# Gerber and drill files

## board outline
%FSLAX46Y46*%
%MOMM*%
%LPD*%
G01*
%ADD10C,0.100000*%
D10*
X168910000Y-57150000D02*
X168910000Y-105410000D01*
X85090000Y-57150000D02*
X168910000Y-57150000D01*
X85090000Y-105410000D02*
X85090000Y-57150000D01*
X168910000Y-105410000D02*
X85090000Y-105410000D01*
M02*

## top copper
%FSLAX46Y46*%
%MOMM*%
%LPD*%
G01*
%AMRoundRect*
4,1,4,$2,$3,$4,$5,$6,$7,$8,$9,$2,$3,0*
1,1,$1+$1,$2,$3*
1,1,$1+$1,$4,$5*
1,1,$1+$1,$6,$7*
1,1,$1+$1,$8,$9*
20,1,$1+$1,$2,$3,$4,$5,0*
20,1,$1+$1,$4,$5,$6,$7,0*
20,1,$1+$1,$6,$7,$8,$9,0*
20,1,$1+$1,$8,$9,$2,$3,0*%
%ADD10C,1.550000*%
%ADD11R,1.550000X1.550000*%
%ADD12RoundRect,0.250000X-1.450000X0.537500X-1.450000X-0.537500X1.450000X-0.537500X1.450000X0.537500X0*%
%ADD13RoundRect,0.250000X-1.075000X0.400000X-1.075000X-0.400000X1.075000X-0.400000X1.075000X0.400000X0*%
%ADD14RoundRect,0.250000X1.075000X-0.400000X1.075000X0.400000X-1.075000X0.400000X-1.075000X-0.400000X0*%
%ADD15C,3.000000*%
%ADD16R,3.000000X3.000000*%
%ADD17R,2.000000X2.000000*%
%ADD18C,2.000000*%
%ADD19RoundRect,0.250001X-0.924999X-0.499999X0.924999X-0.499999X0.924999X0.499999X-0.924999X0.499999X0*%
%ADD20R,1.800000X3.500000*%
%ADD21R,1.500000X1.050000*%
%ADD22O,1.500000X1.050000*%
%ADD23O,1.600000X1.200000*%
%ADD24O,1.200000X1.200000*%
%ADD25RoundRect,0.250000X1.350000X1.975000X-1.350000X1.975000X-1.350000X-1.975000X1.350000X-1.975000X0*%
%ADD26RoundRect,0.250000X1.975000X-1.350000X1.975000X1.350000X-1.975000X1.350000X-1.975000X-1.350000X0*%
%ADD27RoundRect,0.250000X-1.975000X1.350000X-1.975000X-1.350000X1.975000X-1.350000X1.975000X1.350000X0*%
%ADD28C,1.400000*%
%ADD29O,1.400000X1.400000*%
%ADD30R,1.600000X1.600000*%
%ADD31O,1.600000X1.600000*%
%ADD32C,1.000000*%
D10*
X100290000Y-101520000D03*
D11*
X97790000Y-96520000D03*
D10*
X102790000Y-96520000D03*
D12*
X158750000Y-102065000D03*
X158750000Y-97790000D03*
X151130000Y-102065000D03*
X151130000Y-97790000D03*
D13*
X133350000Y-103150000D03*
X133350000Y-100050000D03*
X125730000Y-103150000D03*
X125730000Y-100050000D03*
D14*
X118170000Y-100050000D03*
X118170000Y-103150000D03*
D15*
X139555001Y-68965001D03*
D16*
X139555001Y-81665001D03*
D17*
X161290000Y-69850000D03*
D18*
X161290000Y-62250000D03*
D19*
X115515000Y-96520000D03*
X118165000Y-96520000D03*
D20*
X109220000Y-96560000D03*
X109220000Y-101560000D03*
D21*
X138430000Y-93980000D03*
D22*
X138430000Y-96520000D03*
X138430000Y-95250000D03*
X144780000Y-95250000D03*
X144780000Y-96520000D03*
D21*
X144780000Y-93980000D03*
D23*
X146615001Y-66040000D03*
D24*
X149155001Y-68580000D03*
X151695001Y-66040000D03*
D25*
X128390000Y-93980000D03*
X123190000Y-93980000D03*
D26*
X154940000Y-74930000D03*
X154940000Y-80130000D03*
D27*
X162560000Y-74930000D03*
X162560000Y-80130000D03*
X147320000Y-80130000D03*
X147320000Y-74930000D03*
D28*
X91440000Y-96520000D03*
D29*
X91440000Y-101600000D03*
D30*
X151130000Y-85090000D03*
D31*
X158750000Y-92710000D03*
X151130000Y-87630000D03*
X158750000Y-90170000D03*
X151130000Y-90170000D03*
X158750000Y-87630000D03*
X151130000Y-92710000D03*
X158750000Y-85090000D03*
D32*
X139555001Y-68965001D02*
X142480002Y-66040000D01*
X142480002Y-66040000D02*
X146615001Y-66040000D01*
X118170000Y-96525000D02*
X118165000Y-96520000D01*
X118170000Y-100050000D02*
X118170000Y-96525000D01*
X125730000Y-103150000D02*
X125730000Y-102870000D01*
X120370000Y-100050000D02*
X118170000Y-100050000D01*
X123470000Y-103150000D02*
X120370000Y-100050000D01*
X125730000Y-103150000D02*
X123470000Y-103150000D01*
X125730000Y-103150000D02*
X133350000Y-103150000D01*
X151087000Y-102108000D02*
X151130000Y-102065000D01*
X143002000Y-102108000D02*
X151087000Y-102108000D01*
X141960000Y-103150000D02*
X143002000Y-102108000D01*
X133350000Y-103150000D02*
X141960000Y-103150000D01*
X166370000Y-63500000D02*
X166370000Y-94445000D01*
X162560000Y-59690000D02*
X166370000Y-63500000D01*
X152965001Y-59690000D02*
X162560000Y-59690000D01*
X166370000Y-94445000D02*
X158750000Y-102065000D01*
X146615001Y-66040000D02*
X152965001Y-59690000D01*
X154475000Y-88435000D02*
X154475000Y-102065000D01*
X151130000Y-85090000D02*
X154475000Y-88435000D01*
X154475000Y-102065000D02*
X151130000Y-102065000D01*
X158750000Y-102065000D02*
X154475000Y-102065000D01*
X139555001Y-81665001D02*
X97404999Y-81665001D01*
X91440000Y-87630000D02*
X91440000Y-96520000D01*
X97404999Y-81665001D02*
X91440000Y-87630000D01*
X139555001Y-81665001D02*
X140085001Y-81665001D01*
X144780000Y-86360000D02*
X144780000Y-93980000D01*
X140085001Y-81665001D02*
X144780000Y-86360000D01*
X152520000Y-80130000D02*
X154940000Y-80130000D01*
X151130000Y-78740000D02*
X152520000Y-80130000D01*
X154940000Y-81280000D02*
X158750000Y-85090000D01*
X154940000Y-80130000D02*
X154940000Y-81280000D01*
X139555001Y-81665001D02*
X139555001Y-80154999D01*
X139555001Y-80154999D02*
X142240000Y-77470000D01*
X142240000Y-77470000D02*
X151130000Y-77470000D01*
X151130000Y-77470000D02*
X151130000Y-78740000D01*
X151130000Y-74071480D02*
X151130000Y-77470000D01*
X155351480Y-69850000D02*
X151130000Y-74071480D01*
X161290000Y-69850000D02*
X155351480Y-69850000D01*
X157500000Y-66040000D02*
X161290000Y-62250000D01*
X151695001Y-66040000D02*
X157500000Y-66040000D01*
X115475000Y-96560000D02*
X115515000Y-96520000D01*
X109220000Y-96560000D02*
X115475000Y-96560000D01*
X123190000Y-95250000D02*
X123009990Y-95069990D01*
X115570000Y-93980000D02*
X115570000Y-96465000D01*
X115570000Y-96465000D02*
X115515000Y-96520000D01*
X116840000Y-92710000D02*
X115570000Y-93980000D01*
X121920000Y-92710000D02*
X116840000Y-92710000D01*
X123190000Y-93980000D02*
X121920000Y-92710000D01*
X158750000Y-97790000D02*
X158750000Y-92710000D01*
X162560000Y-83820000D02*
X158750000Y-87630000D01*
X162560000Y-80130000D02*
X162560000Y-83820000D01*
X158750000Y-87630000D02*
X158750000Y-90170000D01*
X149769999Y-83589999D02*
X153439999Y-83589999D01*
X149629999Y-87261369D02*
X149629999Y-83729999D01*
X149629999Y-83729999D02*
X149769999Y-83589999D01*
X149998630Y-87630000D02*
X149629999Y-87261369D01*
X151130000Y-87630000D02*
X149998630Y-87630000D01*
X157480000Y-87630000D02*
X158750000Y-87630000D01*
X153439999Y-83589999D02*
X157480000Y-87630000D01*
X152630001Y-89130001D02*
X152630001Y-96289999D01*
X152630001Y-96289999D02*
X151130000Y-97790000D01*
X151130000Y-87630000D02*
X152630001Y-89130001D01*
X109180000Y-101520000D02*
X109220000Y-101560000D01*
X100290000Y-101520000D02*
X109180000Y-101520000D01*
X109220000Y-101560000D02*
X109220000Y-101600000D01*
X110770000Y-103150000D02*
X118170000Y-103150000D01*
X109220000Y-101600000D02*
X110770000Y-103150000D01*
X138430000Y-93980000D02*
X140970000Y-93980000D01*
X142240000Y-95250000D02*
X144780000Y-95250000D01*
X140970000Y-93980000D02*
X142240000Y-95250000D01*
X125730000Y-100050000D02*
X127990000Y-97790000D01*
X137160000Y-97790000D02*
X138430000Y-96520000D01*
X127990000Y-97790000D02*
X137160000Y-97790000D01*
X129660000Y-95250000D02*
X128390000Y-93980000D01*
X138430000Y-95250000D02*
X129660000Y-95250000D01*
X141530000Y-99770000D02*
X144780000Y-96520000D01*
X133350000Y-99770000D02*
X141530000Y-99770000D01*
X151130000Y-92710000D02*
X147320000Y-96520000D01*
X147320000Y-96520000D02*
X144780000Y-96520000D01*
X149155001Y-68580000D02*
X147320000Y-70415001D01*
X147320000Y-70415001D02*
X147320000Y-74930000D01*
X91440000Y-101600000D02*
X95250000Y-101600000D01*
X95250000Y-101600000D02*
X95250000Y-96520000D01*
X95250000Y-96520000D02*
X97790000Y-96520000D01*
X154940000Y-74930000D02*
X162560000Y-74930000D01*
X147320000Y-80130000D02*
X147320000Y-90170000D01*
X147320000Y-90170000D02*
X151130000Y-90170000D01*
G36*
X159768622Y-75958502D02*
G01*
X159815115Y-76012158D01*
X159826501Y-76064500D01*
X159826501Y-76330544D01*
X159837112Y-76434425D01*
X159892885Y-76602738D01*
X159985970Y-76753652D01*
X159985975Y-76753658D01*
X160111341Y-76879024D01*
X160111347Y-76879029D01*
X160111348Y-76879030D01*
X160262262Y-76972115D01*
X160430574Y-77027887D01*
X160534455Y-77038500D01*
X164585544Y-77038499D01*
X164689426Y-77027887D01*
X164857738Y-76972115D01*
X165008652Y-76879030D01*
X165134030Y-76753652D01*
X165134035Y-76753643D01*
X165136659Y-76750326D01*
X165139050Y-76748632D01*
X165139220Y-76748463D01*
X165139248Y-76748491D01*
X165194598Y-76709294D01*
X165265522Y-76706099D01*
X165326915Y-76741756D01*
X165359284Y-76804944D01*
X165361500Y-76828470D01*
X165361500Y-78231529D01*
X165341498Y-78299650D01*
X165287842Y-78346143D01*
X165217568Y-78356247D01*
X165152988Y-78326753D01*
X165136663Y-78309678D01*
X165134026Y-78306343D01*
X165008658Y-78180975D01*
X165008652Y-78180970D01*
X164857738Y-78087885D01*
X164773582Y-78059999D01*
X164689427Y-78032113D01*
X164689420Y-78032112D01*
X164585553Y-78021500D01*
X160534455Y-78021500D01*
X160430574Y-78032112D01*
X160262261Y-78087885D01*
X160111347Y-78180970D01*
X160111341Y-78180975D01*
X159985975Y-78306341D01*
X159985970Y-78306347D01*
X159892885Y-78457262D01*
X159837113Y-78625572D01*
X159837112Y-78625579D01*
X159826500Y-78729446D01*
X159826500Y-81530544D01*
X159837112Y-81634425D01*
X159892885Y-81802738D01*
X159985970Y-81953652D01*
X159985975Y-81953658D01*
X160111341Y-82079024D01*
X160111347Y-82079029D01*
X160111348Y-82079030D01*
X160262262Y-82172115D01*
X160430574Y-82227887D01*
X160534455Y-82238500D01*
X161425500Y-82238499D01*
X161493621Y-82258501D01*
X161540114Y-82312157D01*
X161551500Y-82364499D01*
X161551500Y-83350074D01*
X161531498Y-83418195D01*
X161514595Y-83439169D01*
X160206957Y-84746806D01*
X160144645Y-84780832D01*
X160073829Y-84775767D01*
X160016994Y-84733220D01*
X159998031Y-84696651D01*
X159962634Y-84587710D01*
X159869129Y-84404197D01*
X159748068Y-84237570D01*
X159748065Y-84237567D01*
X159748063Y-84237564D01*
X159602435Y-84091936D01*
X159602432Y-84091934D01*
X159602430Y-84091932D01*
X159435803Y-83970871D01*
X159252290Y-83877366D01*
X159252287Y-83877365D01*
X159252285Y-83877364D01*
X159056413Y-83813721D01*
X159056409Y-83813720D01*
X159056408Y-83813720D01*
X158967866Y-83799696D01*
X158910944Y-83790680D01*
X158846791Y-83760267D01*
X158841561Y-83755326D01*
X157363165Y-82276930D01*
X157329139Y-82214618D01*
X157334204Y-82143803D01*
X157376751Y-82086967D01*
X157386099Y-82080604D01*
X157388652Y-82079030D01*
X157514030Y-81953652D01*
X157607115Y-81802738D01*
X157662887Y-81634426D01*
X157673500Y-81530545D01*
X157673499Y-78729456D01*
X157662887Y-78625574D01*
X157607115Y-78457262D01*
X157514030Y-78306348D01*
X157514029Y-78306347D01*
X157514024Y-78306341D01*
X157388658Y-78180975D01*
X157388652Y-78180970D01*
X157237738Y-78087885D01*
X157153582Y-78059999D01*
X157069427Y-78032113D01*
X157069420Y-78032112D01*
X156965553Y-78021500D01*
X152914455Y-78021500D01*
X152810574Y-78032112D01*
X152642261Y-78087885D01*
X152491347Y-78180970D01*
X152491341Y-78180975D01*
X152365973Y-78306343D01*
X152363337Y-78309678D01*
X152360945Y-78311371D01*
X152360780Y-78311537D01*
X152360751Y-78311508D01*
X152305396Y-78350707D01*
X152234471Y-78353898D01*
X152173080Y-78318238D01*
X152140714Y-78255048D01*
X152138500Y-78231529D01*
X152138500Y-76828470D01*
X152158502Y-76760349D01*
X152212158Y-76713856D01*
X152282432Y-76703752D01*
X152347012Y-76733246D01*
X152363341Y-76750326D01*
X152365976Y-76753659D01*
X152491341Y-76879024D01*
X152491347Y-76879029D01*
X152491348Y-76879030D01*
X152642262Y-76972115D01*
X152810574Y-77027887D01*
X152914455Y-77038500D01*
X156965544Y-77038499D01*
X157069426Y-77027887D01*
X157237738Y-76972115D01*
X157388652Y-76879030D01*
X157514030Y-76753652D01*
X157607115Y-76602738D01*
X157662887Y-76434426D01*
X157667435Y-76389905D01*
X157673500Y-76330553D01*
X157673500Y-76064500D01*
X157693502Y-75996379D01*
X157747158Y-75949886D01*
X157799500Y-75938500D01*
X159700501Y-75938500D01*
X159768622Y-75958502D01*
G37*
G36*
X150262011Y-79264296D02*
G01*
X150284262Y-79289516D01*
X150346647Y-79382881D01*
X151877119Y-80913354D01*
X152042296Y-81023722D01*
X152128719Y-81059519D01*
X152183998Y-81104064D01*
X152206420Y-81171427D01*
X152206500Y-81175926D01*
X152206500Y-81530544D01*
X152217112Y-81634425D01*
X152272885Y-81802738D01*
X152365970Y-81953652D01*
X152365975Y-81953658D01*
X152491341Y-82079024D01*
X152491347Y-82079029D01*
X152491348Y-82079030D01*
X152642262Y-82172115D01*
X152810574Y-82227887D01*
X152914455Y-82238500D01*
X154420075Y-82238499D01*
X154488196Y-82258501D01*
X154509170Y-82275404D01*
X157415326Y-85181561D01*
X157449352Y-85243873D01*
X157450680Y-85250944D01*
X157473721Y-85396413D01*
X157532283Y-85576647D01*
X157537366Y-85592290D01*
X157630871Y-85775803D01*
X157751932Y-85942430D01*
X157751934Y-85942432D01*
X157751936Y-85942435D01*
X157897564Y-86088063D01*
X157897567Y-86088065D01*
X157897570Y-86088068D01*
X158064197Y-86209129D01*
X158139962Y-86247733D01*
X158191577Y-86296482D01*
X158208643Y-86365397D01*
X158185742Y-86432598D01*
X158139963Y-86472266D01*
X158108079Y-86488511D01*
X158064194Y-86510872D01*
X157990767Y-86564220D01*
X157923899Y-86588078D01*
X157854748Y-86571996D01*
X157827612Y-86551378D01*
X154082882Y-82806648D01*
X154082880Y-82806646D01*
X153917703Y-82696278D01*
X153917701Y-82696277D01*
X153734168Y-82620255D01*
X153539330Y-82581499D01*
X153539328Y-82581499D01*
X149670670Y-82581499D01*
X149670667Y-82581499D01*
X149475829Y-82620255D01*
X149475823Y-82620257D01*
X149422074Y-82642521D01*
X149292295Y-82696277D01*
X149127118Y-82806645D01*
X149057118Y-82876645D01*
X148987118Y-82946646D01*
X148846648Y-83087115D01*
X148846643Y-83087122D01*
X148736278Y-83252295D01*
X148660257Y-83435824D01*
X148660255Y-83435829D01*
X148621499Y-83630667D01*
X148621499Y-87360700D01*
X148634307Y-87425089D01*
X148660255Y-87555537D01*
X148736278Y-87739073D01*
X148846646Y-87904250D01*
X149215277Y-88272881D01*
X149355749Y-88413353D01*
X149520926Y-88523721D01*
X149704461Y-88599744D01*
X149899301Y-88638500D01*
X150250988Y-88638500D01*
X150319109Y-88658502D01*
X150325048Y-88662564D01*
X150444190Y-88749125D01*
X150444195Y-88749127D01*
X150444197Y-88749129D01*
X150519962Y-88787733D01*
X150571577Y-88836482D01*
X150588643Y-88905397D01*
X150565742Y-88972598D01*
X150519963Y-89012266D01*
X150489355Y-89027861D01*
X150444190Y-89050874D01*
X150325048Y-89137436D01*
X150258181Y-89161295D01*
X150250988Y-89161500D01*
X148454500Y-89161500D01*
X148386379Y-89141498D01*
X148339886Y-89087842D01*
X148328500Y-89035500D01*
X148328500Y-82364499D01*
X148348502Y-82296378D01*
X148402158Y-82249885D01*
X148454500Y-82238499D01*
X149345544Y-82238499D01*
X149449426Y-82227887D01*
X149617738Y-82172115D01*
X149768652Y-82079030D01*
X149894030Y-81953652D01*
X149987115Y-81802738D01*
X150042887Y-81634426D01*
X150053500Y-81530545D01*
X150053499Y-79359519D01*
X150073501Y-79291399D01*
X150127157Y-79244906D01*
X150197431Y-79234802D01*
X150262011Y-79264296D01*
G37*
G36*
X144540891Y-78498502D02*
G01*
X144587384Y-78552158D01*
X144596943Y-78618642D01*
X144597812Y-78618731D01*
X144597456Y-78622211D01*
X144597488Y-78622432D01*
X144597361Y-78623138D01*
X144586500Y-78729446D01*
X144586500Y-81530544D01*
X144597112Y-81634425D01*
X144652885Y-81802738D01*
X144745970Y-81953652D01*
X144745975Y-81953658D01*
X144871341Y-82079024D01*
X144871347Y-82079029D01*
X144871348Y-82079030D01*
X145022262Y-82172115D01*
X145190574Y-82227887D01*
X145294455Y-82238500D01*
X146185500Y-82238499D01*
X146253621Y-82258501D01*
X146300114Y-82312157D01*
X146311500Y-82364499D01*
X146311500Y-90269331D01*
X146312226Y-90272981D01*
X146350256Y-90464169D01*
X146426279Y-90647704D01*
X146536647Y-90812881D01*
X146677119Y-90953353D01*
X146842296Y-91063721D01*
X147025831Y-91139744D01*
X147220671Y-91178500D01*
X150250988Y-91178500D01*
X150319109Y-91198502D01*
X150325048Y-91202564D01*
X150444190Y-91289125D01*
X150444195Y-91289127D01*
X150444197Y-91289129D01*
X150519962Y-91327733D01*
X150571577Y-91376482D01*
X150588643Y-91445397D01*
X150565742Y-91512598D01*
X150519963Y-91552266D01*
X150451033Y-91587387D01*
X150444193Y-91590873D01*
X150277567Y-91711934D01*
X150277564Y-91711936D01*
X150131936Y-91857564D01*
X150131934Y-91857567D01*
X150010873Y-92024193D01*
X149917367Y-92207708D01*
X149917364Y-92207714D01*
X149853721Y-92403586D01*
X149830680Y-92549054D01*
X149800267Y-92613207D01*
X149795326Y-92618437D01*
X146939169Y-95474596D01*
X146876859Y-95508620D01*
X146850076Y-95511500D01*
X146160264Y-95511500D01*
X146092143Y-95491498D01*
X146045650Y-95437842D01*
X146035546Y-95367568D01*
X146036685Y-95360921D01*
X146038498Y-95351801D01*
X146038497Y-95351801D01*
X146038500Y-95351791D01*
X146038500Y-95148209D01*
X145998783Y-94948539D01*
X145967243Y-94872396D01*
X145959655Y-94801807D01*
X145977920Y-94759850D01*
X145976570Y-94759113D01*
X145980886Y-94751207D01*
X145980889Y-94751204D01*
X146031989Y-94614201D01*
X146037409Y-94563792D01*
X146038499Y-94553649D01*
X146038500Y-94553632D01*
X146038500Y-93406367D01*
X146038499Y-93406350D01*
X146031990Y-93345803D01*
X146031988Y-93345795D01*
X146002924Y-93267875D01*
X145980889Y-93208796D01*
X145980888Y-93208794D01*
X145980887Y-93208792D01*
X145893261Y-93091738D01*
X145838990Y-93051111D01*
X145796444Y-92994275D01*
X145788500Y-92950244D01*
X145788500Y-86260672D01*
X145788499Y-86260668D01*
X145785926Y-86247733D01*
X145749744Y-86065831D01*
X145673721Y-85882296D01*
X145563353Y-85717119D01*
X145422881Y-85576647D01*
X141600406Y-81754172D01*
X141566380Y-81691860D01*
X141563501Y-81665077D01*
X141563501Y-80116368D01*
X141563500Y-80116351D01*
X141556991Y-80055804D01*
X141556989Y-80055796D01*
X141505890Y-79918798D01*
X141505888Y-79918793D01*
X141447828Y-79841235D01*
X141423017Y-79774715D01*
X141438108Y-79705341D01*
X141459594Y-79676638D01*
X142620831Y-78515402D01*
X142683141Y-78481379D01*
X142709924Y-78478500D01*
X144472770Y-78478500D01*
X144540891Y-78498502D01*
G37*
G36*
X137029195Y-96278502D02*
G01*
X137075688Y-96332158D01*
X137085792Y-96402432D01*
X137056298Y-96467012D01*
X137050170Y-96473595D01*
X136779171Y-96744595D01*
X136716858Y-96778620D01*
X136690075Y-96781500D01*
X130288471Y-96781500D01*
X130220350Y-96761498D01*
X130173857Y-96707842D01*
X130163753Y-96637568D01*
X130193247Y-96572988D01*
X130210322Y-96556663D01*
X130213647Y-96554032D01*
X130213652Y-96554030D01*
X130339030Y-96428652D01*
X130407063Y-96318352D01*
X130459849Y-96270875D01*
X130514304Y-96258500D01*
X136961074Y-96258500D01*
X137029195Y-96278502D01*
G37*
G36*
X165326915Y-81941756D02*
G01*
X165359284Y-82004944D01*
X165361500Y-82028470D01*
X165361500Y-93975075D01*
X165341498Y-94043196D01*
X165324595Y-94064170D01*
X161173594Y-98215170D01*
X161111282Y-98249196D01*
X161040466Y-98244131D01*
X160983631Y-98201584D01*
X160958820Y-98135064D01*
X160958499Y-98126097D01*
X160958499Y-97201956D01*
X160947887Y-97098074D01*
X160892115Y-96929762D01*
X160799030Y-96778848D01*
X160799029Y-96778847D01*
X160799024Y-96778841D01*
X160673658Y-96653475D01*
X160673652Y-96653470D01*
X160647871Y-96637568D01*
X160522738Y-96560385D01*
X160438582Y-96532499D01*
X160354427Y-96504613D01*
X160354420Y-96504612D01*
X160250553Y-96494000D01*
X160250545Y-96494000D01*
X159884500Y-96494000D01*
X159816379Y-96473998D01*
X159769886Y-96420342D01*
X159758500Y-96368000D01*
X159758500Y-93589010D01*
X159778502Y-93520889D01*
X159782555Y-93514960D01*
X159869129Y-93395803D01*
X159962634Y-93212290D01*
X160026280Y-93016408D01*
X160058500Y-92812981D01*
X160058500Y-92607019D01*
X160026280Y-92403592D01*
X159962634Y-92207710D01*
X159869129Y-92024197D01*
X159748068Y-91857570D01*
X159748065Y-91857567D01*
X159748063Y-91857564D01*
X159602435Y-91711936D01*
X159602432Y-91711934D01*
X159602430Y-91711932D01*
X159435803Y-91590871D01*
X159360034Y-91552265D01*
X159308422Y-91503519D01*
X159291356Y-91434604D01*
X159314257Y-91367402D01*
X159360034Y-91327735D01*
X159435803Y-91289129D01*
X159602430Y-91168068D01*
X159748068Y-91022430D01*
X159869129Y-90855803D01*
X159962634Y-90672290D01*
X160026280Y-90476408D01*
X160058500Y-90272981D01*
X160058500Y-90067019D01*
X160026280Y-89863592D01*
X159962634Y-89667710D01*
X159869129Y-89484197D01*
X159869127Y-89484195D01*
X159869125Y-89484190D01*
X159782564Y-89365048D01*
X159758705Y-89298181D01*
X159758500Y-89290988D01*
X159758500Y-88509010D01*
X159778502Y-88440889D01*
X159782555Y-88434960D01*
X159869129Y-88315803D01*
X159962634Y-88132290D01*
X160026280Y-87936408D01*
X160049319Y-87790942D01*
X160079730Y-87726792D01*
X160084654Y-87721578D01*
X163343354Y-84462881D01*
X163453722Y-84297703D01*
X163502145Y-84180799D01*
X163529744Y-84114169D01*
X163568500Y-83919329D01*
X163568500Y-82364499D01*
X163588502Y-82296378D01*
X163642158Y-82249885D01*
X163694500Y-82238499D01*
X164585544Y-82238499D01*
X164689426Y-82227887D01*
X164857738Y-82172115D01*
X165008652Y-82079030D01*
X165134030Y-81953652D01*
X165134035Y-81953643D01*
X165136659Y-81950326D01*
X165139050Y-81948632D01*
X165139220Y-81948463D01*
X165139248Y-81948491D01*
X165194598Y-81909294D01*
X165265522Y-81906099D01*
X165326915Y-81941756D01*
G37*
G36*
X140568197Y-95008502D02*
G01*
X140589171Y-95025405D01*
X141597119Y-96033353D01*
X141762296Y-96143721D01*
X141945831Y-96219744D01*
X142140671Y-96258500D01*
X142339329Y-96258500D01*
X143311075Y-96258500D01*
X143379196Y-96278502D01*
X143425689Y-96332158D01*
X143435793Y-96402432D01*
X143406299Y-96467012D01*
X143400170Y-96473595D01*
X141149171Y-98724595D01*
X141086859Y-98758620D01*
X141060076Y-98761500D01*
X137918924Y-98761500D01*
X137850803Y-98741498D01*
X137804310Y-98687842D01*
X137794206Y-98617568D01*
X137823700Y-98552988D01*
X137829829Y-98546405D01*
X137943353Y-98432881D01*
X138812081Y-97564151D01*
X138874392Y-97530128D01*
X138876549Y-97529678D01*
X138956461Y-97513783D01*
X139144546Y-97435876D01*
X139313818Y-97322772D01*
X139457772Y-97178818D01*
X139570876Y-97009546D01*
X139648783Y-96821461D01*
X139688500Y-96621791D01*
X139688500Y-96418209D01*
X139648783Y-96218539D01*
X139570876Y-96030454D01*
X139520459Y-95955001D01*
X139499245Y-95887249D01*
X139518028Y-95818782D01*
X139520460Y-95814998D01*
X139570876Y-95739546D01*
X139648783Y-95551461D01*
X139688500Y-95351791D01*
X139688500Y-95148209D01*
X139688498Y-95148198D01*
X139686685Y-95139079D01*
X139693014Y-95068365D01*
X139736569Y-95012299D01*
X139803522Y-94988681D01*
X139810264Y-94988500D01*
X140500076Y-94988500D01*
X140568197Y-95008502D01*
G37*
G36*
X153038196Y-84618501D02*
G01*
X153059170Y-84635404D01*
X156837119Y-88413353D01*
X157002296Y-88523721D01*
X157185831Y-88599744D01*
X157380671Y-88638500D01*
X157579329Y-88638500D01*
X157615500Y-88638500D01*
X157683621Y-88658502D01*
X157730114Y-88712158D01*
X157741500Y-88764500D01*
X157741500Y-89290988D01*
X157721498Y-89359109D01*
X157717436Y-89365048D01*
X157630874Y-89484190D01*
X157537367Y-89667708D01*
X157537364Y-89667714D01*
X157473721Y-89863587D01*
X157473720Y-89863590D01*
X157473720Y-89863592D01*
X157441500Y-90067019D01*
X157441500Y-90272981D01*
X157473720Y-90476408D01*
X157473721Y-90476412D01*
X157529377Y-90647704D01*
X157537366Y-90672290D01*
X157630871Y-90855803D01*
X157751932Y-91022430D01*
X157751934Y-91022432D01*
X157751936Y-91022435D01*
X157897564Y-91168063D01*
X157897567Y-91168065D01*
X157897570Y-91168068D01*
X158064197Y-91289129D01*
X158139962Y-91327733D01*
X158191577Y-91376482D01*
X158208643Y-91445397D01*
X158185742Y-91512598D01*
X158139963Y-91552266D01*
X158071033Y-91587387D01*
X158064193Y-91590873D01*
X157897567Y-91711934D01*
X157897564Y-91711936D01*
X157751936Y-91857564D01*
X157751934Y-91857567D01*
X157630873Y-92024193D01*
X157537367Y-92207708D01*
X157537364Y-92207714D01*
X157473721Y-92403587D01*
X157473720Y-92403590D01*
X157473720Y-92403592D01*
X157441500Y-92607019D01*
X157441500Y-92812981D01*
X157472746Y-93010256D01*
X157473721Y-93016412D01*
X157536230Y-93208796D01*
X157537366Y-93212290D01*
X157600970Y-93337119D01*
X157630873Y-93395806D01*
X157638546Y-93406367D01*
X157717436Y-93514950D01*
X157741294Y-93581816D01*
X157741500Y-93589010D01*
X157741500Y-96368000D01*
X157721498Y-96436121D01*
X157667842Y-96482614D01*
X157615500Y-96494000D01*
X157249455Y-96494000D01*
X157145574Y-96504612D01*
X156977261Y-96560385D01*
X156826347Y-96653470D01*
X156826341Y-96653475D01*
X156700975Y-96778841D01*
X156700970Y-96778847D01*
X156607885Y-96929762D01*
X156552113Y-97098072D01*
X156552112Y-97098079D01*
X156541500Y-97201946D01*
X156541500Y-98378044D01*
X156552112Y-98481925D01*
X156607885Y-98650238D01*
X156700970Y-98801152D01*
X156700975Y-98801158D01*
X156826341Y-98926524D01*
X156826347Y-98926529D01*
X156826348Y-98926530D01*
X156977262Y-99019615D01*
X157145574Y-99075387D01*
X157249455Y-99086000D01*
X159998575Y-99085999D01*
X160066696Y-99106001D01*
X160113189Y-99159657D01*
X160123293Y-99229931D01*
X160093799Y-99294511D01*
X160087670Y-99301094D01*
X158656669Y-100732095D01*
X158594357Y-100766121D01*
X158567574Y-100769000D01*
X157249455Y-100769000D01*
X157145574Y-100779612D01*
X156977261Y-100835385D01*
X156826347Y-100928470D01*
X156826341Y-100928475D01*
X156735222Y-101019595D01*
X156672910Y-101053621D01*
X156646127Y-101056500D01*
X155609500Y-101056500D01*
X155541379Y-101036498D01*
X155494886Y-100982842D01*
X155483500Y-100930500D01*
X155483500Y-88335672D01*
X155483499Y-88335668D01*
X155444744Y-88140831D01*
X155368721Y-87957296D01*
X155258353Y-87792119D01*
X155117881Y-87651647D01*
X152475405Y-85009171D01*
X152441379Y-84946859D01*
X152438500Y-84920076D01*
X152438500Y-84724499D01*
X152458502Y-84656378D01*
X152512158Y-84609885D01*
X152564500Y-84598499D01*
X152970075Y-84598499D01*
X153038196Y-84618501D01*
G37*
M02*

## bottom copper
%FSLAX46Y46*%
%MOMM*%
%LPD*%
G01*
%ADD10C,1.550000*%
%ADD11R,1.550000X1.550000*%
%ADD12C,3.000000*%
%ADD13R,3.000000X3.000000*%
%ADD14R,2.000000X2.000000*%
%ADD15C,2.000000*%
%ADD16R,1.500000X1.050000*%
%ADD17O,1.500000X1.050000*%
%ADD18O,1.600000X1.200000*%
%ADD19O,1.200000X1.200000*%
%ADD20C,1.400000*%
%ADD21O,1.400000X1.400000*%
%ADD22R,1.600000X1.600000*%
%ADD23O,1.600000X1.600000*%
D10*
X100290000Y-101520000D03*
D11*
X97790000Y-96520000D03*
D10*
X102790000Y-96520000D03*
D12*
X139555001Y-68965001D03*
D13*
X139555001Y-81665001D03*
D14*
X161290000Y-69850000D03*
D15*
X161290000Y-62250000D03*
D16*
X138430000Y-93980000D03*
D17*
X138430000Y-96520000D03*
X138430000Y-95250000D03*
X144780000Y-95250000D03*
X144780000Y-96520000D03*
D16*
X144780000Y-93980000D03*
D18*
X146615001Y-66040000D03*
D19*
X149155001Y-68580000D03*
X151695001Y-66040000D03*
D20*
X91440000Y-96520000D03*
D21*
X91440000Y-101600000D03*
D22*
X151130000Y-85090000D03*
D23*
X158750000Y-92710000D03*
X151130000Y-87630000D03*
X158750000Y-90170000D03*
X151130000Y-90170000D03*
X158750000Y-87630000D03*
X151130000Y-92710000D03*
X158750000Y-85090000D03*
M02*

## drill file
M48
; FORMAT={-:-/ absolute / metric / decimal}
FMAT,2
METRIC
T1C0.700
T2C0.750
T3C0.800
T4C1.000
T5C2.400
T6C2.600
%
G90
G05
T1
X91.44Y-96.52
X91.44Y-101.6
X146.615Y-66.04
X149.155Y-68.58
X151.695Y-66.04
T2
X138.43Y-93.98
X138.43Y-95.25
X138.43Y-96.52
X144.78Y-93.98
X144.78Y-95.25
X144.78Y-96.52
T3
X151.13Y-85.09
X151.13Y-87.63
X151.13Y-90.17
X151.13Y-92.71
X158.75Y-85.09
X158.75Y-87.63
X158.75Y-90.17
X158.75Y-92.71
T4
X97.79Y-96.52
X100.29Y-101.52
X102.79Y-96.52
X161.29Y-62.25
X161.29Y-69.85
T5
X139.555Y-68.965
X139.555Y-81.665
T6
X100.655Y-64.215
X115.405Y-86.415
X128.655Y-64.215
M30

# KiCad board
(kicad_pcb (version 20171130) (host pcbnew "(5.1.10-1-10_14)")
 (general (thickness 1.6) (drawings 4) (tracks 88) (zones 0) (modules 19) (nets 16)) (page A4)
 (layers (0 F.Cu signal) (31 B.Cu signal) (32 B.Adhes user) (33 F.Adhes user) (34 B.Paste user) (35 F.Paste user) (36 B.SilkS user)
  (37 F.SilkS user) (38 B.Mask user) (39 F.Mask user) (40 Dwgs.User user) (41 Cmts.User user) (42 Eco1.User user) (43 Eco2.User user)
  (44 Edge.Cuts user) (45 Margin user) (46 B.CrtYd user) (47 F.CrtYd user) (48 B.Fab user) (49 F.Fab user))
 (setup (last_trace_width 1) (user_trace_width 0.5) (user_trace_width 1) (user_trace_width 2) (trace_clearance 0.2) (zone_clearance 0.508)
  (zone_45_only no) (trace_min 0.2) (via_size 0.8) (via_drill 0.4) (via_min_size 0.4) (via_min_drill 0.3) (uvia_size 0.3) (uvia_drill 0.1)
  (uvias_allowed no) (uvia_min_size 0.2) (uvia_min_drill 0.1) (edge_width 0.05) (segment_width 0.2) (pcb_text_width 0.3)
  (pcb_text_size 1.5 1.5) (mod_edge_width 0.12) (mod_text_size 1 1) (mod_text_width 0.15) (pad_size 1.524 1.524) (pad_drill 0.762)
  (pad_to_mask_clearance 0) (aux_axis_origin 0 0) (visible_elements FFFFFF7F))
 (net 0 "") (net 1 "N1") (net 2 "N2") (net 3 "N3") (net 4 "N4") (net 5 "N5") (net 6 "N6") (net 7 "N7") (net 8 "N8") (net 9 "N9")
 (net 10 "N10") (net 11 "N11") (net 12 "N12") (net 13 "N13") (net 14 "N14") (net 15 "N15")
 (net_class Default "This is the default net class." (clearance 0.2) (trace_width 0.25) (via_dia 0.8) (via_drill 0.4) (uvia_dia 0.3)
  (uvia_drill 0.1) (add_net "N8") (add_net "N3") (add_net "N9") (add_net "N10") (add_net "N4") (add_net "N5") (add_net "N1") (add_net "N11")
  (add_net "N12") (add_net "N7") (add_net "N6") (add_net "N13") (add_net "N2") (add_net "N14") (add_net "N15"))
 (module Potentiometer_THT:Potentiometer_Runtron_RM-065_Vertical (layer F.Cu) (at 97.79 96.52)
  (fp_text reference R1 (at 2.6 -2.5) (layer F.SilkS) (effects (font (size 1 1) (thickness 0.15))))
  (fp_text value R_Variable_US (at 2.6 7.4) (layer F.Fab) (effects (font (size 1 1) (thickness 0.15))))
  (pad 2 thru_hole circle (at 2.5 5) (size 1.55 1.55) (drill 1) (layers *.Cu *.Mask) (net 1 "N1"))
  (pad 1 thru_hole rect (at 0 0) (size 1.55 1.55) (drill 1) (layers *.Cu *.Mask) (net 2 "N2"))
  (pad 3 thru_hole circle (at 5 0) (size 1.55 1.55) (drill 1) (layers *.Cu *.Mask)))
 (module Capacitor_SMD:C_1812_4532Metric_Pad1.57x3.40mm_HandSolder (layer F.Cu) (at 158.75 99.9275 270)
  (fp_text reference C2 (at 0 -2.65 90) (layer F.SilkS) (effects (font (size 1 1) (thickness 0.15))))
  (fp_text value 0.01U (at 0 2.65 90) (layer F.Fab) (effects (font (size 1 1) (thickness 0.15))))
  (pad 2 smd roundrect (at 2.1375 0 270) (size 1.575 3.4) (layers F.Cu F.Paste F.Mask) (roundrect_rratio 0.15873) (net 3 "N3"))
  (pad 1 smd roundrect (at -2.1375 0 270) (size 1.575 3.4) (layers F.Cu F.Paste F.Mask) (roundrect_rratio 0.15873) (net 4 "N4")))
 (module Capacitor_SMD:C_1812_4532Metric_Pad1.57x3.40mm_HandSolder (layer F.Cu) (at 151.13 99.9275 270)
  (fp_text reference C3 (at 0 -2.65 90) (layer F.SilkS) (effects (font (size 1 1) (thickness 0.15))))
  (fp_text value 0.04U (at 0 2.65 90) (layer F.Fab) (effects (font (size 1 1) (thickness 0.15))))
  (pad 2 smd roundrect (at 2.1375 0 270) (size 1.575 3.4) (layers F.Cu F.Paste F.Mask) (roundrect_rratio 0.15873) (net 3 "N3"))
  (pad 1 smd roundrect (at -2.1375 0 270) (size 1.575 3.4) (layers F.Cu F.Paste F.Mask) (roundrect_rratio 0.15873) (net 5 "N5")))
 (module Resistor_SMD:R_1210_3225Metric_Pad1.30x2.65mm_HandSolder (layer F.Cu) (at 133.35 101.6 270)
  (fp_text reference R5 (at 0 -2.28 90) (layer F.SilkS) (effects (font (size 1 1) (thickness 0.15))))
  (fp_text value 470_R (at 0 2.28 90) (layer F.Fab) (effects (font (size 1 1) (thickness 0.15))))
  (pad 2 smd roundrect (at 1.55 0 270) (size 1.3 2.65) (layers F.Cu F.Paste F.Mask) (roundrect_rratio 0.192308) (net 3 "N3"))
  (pad 1 smd roundrect (at -1.55 0 270) (size 1.3 2.65) (layers F.Cu F.Paste F.Mask) (roundrect_rratio 0.192308) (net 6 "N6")))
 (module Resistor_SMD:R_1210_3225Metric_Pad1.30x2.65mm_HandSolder (layer F.Cu) (at 125.73 101.6 270)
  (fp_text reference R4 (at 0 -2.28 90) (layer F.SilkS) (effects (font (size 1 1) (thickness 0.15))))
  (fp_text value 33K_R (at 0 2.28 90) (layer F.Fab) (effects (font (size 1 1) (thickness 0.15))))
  (pad 2 smd roundrect (at 1.55 0 270) (size 1.3 2.65) (layers F.Cu F.Paste F.Mask) (roundrect_rratio 0.192308) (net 3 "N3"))
  (pad 1 smd roundrect (at -1.55 0 270) (size 1.3 2.65) (layers F.Cu F.Paste F.Mask) (roundrect_rratio 0.192308) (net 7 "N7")))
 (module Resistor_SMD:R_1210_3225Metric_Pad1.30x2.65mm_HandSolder (layer F.Cu) (at 118.17 101.6 90)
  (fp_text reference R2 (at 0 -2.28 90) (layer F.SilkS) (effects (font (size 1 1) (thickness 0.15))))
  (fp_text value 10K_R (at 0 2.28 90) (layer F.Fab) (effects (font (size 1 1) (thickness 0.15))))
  (pad 2 smd roundrect (at 1.55 0 90) (size 1.3 2.65) (layers F.Cu F.Paste F.Mask) (roundrect_rratio 0.192308) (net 3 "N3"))
  (pad 1 smd roundrect (at -1.55 0 90) (size 1.3 2.65) (layers F.Cu F.Paste F.Mask) (roundrect_rratio 0.192308) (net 1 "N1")))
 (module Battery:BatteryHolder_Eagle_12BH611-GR (layer F.Cu) (at 139.555001 81.665001)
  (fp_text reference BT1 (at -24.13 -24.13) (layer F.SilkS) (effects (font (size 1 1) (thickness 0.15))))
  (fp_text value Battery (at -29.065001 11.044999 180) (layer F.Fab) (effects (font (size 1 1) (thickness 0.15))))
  (pad 2 thru_hole circle (at 0 -12.7) (size 3 3) (drill 2.4) (layers *.Cu *.Mask) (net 3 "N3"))
  (pad 1 thru_hole rect (at 0 0) (size 3 3) (drill 2.4) (layers *.Cu *.Mask) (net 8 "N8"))
  (pad "" np_thru_hole circle (at -10.9 -17.45) (size 2.6 2.6) (drill 2.6) (layers *.Cu *.Mask))
  (pad "" np_thru_hole circle (at -38.9 -17.45) (size 2.6 2.6) (drill 2.6) (layers *.Cu *.Mask))
  (pad "" np_thru_hole circle (at -24.15 4.75) (size 2.6 2.6) (drill 2.6) (layers *.Cu *.Mask)))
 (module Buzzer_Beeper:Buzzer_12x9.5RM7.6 (layer F.Cu) (at 161.29 69.85 90)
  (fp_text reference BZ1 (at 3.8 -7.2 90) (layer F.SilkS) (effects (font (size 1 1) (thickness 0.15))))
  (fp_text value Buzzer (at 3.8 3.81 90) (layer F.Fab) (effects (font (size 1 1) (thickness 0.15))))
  (pad 1 thru_hole rect (at 0 0 90) (size 2 2) (drill 1) (layers *.Cu *.Mask) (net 8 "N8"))
  (pad 2 thru_hole circle (at 7.6 0 90) (size 2 2) (drill 1) (layers *.Cu *.Mask) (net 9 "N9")))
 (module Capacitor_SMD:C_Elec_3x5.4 (layer F.Cu) (at 116.84 96.52)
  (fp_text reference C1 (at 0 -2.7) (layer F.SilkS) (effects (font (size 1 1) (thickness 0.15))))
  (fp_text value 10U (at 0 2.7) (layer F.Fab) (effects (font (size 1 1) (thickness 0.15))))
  (pad 1 smd roundrect (at -1.325 0) (size 2.35 1.5) (layers F.Cu F.Paste F.Mask) (roundrect_rratio 0.166667) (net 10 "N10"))
  (pad 2 smd roundrect (at 1.325 0) (size 2.35 1.5) (layers F.Cu F.Paste F.Mask) (roundrect_rratio 0.166667) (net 3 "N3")))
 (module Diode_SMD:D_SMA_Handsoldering (layer F.Cu) (at 109.22 99.06 270)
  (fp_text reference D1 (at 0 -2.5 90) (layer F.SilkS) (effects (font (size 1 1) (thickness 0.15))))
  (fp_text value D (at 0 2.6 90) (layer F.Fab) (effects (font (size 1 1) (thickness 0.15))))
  (pad 1 smd rect (at -2.5 0 270) (size 3.5 1.8) (layers F.Cu F.Paste F.Mask) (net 10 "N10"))
  (pad 2 smd rect (at 2.5 0 270) (size 3.5 1.8) (layers F.Cu F.Paste F.Mask) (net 1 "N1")))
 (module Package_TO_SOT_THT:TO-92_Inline (layer F.Cu) (at 138.43 93.98 270)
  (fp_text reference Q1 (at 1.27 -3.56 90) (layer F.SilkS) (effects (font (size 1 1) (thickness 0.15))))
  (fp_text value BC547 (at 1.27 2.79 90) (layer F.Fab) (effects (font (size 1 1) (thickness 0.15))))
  (pad 1 thru_hole rect (at 0 0 270) (size 1.05 1.5) (drill 0.75) (layers *.Cu *.Mask) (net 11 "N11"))
  (pad 3 thru_hole oval (at 2.54 0 270) (size 1.05 1.5) (drill 0.75) (layers *.Cu *.Mask) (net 7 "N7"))
  (pad 2 thru_hole oval (at 1.27 0 270) (size 1.05 1.5) (drill 0.75) (layers *.Cu *.Mask) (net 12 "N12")))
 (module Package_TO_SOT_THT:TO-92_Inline (layer F.Cu) (at 144.78 93.98 270)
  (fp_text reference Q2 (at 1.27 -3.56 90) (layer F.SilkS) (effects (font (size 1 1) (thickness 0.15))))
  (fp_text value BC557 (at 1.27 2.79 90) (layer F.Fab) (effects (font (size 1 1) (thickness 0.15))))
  (pad 2 thru_hole oval (at 1.27 0 270) (size 1.05 1.5) (drill 0.75) (layers *.Cu *.Mask) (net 11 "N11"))
  (pad 3 thru_hole oval (at 2.54 0 270) (size 1.05 1.5) (drill 0.75) (layers *.Cu *.Mask) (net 6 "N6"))
  (pad 1 thru_hole rect (at 0 0 270) (size 1.05 1.5) (drill 0.75) (layers *.Cu *.Mask) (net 8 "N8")))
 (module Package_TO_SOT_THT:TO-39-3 (layer F.Cu) (at 146.615001 66.04)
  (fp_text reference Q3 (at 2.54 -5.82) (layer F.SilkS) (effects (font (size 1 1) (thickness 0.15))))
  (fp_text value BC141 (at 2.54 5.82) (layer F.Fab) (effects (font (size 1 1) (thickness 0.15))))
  (pad 1 thru_hole oval (at 0 0) (size 1.6 1.2) (drill 0.7) (layers *.Cu *.Mask) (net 3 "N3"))
  (pad 2 thru_hole oval (at 2.54 2.54) (size 1.2 1.2) (drill 0.7) (layers *.Cu *.Mask) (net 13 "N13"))
  (pad 3 thru_hole oval (at 5.08 0) (size 1.2 1.2) (drill 0.7) (layers *.Cu *.Mask) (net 9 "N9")))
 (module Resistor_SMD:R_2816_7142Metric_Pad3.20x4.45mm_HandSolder (layer F.Cu) (at 125.79 93.98 180)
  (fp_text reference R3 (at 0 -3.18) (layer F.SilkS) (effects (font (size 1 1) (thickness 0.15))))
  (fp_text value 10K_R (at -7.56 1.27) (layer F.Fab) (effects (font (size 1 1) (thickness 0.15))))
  (pad 1 smd roundrect (at -2.6 0 180) (size 3.2 4.45) (layers F.Cu F.Paste F.Mask) (roundrect_rratio 0.078125) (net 12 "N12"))
  (pad 2 smd roundrect (at 2.6 0 180) (size 3.2 4.45) (layers F.Cu F.Paste F.Mask) (roundrect_rratio 0.078125) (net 10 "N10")))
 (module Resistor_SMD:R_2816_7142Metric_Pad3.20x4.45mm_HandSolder (layer F.Cu) (at 154.94 77.53 90)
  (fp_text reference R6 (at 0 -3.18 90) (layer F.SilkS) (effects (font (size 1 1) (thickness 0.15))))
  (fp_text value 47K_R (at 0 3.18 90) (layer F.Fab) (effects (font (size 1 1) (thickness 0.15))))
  (pad 2 smd roundrect (at 2.6 0 90) (size 3.2 4.45) (layers F.Cu F.Paste F.Mask) (roundrect_rratio 0.078125) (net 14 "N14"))
  (pad 1 smd roundrect (at -2.6 0 90) (size 3.2 4.45) (layers F.Cu F.Paste F.Mask) (roundrect_rratio 0.078125) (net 8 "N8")))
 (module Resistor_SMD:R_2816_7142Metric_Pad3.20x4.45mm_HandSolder (layer F.Cu) (at 162.56 77.53 270)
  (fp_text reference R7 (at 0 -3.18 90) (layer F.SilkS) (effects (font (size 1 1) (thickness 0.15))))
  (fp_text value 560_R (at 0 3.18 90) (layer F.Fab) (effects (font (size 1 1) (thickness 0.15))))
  (pad 1 smd roundrect (at -2.6 0 270) (size 3.2 4.45) (layers F.Cu F.Paste F.Mask) (roundrect_rratio 0.078125) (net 14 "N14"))
  (pad 2 smd roundrect (at 2.6 0 270) (size 3.2 4.45) (layers F.Cu F.Paste F.Mask) (roundrect_rratio 0.078125) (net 5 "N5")))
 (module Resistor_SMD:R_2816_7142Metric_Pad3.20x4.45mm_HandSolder (layer F.Cu) (at 147.32 77.53 270)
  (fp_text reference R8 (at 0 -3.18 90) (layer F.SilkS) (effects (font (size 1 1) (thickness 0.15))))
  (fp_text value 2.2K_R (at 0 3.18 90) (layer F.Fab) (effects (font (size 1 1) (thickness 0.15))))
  (pad 2 smd roundrect (at 2.6 0 270) (size 3.2 4.45) (layers F.Cu F.Paste F.Mask) (roundrect_rratio 0.078125) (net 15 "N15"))
  (pad 1 smd roundrect (at -2.6 0 270) (size 3.2 4.45) (layers F.Cu F.Paste F.Mask) (roundrect_rratio 0.078125) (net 13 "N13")))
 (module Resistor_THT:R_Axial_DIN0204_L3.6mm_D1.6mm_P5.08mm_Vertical (layer F.Cu) (at 91.44 96.52 270)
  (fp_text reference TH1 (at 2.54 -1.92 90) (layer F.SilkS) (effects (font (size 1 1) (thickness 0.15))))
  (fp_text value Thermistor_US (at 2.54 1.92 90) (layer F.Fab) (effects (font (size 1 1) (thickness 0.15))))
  (pad 1 thru_hole circle (at 0 0 270) (size 1.4 1.4) (drill 0.7) (layers *.Cu *.Mask) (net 8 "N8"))
  (pad 2 thru_hole oval (at 5.08 0 270) (size 1.4 1.4) (drill 0.7) (layers *.Cu *.Mask) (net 2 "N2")))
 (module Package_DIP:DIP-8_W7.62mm (layer F.Cu) (at 151.13 85.09)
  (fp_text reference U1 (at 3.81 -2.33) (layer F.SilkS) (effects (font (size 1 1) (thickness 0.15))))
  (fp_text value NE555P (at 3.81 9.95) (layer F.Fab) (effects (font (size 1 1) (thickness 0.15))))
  (pad 1 thru_hole rect (at 0 0) (size 1.6 1.6) (drill 0.8) (layers *.Cu *.Mask) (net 3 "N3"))
  (pad 5 thru_hole oval (at 7.62 7.62) (size 1.6 1.6) (drill 0.8) (layers *.Cu *.Mask) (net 4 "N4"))
  (pad 2 thru_hole oval (at 0 2.54) (size 1.6 1.6) (drill 0.8) (layers *.Cu *.Mask) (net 5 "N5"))
  (pad 6 thru_hole oval (at 7.62 5.08) (size 1.6 1.6) (drill 0.8) (layers *.Cu *.Mask) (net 5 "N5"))
  (pad 3 thru_hole oval (at 0 5.08) (size 1.6 1.6) (drill 0.8) (layers *.Cu *.Mask) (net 15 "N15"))
  (pad 7 thru_hole oval (at 7.62 2.54) (size 1.6 1.6) (drill 0.8) (layers *.Cu *.Mask) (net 5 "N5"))
  (pad 4 thru_hole oval (at 0 7.62) (size 1.6 1.6) (drill 0.8) (layers *.Cu *.Mask) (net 6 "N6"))
  (pad 8 thru_hole oval (at 7.62 0) (size 1.6 1.6) (drill 0.8) (layers *.Cu *.Mask) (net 8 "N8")))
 (gr_line (start 168.91 57.15) (end 168.91 105.41) (layer Edge.Cuts) (width 0.1))
 (gr_line (start 85.09 57.15) (end 168.91 57.15) (layer Edge.Cuts) (width 0.1))
 (gr_line (start 85.09 105.41) (end 85.09 57.15) (layer Edge.Cuts) (width 0.1))
 (gr_line (start 168.91 105.41) (end 85.09 105.41) (layer Edge.Cuts) (width 0.1))
 (segment (start 139.555001 68.965001) (end 142.480002 66.04) (width 1) (layer F.Cu) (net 3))
 (segment (start 142.480002 66.04) (end 146.615001 66.04) (width 1) (layer F.Cu) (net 3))
 (segment (start 118.17 96.525) (end 118.165 96.52) (width 1) (layer F.Cu) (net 3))
 (segment (start 118.17 100.05) (end 118.17 96.525) (width 1) (layer F.Cu) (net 3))
 (segment (start 125.73 103.15) (end 125.73 102.87) (width 1) (layer F.Cu) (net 3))
 (segment (start 120.37 100.05) (end 118.17 100.05) (width 1) (layer F.Cu) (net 3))
 (segment (start 123.47 103.15) (end 120.37 100.05) (width 1) (layer F.Cu) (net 3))
 (segment (start 125.73 103.15) (end 123.47 103.15) (width 1) (layer F.Cu) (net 3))
 (segment (start 125.73 103.15) (end 133.35 103.15) (width 1) (layer F.Cu) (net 3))
 (segment (start 151.087 102.108) (end 151.13 102.065) (width 1) (layer F.Cu) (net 3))
 (segment (start 143.002 102.108) (end 151.087 102.108) (width 1) (layer F.Cu) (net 3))
 (segment (start 141.96 103.15) (end 143.002 102.108) (width 1) (layer F.Cu) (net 3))
 (segment (start 133.35 103.15) (end 141.96 103.15) (width 1) (layer F.Cu) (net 3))
 (segment (start 166.37 63.5) (end 166.37 94.445) (width 1) (layer F.Cu) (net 3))
 (segment (start 162.56 59.69) (end 166.37 63.5) (width 1) (layer F.Cu) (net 3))
 (segment (start 152.965001 59.69) (end 162.56 59.69) (width 1) (layer F.Cu) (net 3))
 (segment (start 166.37 94.445) (end 158.75 102.065) (width 1) (layer F.Cu) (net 3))
 (segment (start 146.615001 66.04) (end 152.965001 59.69) (width 1) (layer F.Cu) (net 3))
 (segment (start 154.475 88.435) (end 154.475 102.065) (width 1) (layer F.Cu) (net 3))
 (segment (start 151.13 85.09) (end 154.475 88.435) (width 1) (layer F.Cu) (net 3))
 (segment (start 154.475 102.065) (end 151.13 102.065) (width 1) (layer F.Cu) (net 3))
 (segment (start 158.75 102.065) (end 154.475 102.065) (width 1) (layer F.Cu) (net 3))
 (segment (start 139.555001 81.665001) (end 97.404999 81.665001) (width 1) (layer F.Cu) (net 8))
 (segment (start 91.44 87.63) (end 91.44 96.52) (width 1) (layer F.Cu) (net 8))
 (segment (start 97.404999 81.665001) (end 91.44 87.63) (width 1) (layer F.Cu) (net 8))
 (segment (start 139.555001 81.665001) (end 140.085001 81.665001) (width 1) (layer F.Cu) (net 8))
 (segment (start 144.78 86.36) (end 144.78 93.98) (width 1) (layer F.Cu) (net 8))
 (segment (start 140.085001 81.665001) (end 144.78 86.36) (width 1) (layer F.Cu) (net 8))
 (segment (start 152.52 80.13) (end 154.94 80.13) (width 1) (layer F.Cu) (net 8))
 (segment (start 151.13 78.74) (end 152.52 80.13) (width 1) (layer F.Cu) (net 8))
 (segment (start 154.94 81.28) (end 158.75 85.09) (width 1) (layer F.Cu) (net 8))
 (segment (start 154.94 80.13) (end 154.94 81.28) (width 1) (layer F.Cu) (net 8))
 (segment (start 139.555001 81.665001) (end 139.555001 80.154999) (width 1) (layer F.Cu) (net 8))
 (segment (start 139.555001 80.154999) (end 142.24 77.47) (width 1) (layer F.Cu) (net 8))
 (segment (start 142.24 77.47) (end 151.13 77.47) (width 1) (layer F.Cu) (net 8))
 (segment (start 151.13 77.47) (end 151.13 78.74) (width 1) (layer F.Cu) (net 8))
 (segment (start 151.13 74.07148) (end 151.13 77.47) (width 1) (layer F.Cu) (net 8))
 (segment (start 155.35148 69.85) (end 151.13 74.07148) (width 1) (layer F.Cu) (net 8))
 (segment (start 161.29 69.85) (end 155.35148 69.85) (width 1) (layer F.Cu) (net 8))
 (segment (start 157.5 66.04) (end 161.29 62.25) (width 1) (layer F.Cu) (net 9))
 (segment (start 151.695001 66.04) (end 157.5 66.04) (width 1) (layer F.Cu) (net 9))
 (segment (start 115.475 96.56) (end 115.515 96.52) (width 1) (layer F.Cu) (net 10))
 (segment (start 109.22 96.56) (end 115.475 96.56) (width 1) (layer F.Cu) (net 10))
 (segment (start 123.19 95.25) (end 123.00999 95.06999) (width 1) (layer F.Cu) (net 10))
 (segment (start 115.57 93.98) (end 115.57 96.465) (width 1) (layer F.Cu) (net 10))
 (segment (start 115.57 96.465) (end 115.515 96.52) (width 1) (layer F.Cu) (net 10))
 (segment (start 116.84 92.71) (end 115.57 93.98) (width 1) (layer F.Cu) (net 10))
 (segment (start 121.92 92.71) (end 116.84 92.71) (width 1) (layer F.Cu) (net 10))
 (segment (start 123.19 93.98) (end 121.92 92.71) (width 1) (layer F.Cu) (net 10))
 (segment (start 158.75 97.79) (end 158.75 92.71) (width 1) (layer F.Cu) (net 4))
 (segment (start 162.56 83.82) (end 158.75 87.63) (width 1) (layer F.Cu) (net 5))
 (segment (start 162.56 80.13) (end 162.56 83.82) (width 1) (layer F.Cu) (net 5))
 (segment (start 158.75 87.63) (end 158.75 90.17) (width 1) (layer F.Cu) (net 5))
 (segment (start 149.769999 83.589999) (end 153.439999 83.589999) (width 1) (layer F.Cu) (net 5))
 (segment (start 149.629999 87.261369) (end 149.629999 83.729999) (width 1) (layer F.Cu) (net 5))
 (segment (start 149.629999 83.729999) (end 149.769999 83.589999) (width 1) (layer F.Cu) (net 5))
 (segment (start 149.99863 87.63) (end 149.629999 87.261369) (width 1) (layer F.Cu) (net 5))
 (segment (start 151.13 87.63) (end 149.99863 87.63) (width 1) (layer F.Cu) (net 5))
 (segment (start 157.48 87.63) (end 158.75 87.63) (width 1) (layer F.Cu) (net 5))
 (segment (start 153.439999 83.589999) (end 157.48 87.63) (width 1) (layer F.Cu) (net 5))
 (segment (start 152.630001 89.130001) (end 152.630001 96.289999) (width 1) (layer F.Cu) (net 5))
 (segment (start 152.630001 96.289999) (end 151.13 97.79) (width 1) (layer F.Cu) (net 5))
 (segment (start 151.13 87.63) (end 152.630001 89.130001) (width 1) (layer F.Cu) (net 5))
 (segment (start 109.18 101.52) (end 109.22 101.56) (width 1) (layer F.Cu) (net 1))
 (segment (start 100.29 101.52) (end 109.18 101.52) (width 1) (layer F.Cu) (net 1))
 (segment (start 109.22 101.56) (end 109.22 101.6) (width 1) (layer F.Cu) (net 1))
 (segment (start 110.77 103.15) (end 118.17 103.15) (width 1) (layer F.Cu) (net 1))
 (segment (start 109.22 101.6) (end 110.77 103.15) (width 1) (layer F.Cu) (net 1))
 (segment (start 138.43 93.98) (end 140.97 93.98) (width 1) (layer F.Cu) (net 11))
 (segment (start 142.24 95.25) (end 144.78 95.25) (width 1) (layer F.Cu) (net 11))
 (segment (start 140.97 93.98) (end 142.24 95.25) (width 1) (layer F.Cu) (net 11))
 (segment (start 125.73 100.05) (end 127.99 97.79) (width 1) (layer F.Cu) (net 7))
 (segment (start 137.16 97.79) (end 138.43 96.52) (width 1) (layer F.Cu) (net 7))
 (segment (start 127.99 97.79) (end 137.16 97.79) (width 1) (layer F.Cu) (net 7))
 (segment (start 129.66 95.25) (end 128.39 93.98) (width 1) (layer F.Cu) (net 12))
 (segment (start 138.43 95.25) (end 129.66 95.25) (width 1) (layer F.Cu) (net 12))
 (segment (start 141.53 99.77) (end 144.78 96.52) (width 1) (layer F.Cu) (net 6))
 (segment (start 133.35 99.77) (end 141.53 99.77) (width 1) (layer F.Cu) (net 6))
 (segment (start 151.13 92.71) (end 147.32 96.52) (width 1) (layer F.Cu) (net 6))
 (segment (start 147.32 96.52) (end 144.78 96.52) (width 1) (layer F.Cu) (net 6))
 (segment (start 149.155001 68.58) (end 147.32 70.415001) (width 1) (layer F.Cu) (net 13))
 (segment (start 147.32 70.415001) (end 147.32 74.93) (width 1) (layer F.Cu) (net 13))
 (segment (start 91.44 101.6) (end 95.25 101.6) (width 1) (layer F.Cu) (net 2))
 (segment (start 95.25 101.6) (end 95.25 96.52) (width 1) (layer F.Cu) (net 2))
 (segment (start 95.25 96.52) (end 97.79 96.52) (width 1) (layer F.Cu) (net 2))
 (segment (start 154.94 74.93) (end 162.56 74.93) (width 1) (layer F.Cu) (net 14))
 (segment (start 147.32 80.13) (end 147.32 90.17) (width 1) (layer F.Cu) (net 15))
 (segment (start 147.32 90.17) (end 151.13 90.17) (width 1) (layer F.Cu) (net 15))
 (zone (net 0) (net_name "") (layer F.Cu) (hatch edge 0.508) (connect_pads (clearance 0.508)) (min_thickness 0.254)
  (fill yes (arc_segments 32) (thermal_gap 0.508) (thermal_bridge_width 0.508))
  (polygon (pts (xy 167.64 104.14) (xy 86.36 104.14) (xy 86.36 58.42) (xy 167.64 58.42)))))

